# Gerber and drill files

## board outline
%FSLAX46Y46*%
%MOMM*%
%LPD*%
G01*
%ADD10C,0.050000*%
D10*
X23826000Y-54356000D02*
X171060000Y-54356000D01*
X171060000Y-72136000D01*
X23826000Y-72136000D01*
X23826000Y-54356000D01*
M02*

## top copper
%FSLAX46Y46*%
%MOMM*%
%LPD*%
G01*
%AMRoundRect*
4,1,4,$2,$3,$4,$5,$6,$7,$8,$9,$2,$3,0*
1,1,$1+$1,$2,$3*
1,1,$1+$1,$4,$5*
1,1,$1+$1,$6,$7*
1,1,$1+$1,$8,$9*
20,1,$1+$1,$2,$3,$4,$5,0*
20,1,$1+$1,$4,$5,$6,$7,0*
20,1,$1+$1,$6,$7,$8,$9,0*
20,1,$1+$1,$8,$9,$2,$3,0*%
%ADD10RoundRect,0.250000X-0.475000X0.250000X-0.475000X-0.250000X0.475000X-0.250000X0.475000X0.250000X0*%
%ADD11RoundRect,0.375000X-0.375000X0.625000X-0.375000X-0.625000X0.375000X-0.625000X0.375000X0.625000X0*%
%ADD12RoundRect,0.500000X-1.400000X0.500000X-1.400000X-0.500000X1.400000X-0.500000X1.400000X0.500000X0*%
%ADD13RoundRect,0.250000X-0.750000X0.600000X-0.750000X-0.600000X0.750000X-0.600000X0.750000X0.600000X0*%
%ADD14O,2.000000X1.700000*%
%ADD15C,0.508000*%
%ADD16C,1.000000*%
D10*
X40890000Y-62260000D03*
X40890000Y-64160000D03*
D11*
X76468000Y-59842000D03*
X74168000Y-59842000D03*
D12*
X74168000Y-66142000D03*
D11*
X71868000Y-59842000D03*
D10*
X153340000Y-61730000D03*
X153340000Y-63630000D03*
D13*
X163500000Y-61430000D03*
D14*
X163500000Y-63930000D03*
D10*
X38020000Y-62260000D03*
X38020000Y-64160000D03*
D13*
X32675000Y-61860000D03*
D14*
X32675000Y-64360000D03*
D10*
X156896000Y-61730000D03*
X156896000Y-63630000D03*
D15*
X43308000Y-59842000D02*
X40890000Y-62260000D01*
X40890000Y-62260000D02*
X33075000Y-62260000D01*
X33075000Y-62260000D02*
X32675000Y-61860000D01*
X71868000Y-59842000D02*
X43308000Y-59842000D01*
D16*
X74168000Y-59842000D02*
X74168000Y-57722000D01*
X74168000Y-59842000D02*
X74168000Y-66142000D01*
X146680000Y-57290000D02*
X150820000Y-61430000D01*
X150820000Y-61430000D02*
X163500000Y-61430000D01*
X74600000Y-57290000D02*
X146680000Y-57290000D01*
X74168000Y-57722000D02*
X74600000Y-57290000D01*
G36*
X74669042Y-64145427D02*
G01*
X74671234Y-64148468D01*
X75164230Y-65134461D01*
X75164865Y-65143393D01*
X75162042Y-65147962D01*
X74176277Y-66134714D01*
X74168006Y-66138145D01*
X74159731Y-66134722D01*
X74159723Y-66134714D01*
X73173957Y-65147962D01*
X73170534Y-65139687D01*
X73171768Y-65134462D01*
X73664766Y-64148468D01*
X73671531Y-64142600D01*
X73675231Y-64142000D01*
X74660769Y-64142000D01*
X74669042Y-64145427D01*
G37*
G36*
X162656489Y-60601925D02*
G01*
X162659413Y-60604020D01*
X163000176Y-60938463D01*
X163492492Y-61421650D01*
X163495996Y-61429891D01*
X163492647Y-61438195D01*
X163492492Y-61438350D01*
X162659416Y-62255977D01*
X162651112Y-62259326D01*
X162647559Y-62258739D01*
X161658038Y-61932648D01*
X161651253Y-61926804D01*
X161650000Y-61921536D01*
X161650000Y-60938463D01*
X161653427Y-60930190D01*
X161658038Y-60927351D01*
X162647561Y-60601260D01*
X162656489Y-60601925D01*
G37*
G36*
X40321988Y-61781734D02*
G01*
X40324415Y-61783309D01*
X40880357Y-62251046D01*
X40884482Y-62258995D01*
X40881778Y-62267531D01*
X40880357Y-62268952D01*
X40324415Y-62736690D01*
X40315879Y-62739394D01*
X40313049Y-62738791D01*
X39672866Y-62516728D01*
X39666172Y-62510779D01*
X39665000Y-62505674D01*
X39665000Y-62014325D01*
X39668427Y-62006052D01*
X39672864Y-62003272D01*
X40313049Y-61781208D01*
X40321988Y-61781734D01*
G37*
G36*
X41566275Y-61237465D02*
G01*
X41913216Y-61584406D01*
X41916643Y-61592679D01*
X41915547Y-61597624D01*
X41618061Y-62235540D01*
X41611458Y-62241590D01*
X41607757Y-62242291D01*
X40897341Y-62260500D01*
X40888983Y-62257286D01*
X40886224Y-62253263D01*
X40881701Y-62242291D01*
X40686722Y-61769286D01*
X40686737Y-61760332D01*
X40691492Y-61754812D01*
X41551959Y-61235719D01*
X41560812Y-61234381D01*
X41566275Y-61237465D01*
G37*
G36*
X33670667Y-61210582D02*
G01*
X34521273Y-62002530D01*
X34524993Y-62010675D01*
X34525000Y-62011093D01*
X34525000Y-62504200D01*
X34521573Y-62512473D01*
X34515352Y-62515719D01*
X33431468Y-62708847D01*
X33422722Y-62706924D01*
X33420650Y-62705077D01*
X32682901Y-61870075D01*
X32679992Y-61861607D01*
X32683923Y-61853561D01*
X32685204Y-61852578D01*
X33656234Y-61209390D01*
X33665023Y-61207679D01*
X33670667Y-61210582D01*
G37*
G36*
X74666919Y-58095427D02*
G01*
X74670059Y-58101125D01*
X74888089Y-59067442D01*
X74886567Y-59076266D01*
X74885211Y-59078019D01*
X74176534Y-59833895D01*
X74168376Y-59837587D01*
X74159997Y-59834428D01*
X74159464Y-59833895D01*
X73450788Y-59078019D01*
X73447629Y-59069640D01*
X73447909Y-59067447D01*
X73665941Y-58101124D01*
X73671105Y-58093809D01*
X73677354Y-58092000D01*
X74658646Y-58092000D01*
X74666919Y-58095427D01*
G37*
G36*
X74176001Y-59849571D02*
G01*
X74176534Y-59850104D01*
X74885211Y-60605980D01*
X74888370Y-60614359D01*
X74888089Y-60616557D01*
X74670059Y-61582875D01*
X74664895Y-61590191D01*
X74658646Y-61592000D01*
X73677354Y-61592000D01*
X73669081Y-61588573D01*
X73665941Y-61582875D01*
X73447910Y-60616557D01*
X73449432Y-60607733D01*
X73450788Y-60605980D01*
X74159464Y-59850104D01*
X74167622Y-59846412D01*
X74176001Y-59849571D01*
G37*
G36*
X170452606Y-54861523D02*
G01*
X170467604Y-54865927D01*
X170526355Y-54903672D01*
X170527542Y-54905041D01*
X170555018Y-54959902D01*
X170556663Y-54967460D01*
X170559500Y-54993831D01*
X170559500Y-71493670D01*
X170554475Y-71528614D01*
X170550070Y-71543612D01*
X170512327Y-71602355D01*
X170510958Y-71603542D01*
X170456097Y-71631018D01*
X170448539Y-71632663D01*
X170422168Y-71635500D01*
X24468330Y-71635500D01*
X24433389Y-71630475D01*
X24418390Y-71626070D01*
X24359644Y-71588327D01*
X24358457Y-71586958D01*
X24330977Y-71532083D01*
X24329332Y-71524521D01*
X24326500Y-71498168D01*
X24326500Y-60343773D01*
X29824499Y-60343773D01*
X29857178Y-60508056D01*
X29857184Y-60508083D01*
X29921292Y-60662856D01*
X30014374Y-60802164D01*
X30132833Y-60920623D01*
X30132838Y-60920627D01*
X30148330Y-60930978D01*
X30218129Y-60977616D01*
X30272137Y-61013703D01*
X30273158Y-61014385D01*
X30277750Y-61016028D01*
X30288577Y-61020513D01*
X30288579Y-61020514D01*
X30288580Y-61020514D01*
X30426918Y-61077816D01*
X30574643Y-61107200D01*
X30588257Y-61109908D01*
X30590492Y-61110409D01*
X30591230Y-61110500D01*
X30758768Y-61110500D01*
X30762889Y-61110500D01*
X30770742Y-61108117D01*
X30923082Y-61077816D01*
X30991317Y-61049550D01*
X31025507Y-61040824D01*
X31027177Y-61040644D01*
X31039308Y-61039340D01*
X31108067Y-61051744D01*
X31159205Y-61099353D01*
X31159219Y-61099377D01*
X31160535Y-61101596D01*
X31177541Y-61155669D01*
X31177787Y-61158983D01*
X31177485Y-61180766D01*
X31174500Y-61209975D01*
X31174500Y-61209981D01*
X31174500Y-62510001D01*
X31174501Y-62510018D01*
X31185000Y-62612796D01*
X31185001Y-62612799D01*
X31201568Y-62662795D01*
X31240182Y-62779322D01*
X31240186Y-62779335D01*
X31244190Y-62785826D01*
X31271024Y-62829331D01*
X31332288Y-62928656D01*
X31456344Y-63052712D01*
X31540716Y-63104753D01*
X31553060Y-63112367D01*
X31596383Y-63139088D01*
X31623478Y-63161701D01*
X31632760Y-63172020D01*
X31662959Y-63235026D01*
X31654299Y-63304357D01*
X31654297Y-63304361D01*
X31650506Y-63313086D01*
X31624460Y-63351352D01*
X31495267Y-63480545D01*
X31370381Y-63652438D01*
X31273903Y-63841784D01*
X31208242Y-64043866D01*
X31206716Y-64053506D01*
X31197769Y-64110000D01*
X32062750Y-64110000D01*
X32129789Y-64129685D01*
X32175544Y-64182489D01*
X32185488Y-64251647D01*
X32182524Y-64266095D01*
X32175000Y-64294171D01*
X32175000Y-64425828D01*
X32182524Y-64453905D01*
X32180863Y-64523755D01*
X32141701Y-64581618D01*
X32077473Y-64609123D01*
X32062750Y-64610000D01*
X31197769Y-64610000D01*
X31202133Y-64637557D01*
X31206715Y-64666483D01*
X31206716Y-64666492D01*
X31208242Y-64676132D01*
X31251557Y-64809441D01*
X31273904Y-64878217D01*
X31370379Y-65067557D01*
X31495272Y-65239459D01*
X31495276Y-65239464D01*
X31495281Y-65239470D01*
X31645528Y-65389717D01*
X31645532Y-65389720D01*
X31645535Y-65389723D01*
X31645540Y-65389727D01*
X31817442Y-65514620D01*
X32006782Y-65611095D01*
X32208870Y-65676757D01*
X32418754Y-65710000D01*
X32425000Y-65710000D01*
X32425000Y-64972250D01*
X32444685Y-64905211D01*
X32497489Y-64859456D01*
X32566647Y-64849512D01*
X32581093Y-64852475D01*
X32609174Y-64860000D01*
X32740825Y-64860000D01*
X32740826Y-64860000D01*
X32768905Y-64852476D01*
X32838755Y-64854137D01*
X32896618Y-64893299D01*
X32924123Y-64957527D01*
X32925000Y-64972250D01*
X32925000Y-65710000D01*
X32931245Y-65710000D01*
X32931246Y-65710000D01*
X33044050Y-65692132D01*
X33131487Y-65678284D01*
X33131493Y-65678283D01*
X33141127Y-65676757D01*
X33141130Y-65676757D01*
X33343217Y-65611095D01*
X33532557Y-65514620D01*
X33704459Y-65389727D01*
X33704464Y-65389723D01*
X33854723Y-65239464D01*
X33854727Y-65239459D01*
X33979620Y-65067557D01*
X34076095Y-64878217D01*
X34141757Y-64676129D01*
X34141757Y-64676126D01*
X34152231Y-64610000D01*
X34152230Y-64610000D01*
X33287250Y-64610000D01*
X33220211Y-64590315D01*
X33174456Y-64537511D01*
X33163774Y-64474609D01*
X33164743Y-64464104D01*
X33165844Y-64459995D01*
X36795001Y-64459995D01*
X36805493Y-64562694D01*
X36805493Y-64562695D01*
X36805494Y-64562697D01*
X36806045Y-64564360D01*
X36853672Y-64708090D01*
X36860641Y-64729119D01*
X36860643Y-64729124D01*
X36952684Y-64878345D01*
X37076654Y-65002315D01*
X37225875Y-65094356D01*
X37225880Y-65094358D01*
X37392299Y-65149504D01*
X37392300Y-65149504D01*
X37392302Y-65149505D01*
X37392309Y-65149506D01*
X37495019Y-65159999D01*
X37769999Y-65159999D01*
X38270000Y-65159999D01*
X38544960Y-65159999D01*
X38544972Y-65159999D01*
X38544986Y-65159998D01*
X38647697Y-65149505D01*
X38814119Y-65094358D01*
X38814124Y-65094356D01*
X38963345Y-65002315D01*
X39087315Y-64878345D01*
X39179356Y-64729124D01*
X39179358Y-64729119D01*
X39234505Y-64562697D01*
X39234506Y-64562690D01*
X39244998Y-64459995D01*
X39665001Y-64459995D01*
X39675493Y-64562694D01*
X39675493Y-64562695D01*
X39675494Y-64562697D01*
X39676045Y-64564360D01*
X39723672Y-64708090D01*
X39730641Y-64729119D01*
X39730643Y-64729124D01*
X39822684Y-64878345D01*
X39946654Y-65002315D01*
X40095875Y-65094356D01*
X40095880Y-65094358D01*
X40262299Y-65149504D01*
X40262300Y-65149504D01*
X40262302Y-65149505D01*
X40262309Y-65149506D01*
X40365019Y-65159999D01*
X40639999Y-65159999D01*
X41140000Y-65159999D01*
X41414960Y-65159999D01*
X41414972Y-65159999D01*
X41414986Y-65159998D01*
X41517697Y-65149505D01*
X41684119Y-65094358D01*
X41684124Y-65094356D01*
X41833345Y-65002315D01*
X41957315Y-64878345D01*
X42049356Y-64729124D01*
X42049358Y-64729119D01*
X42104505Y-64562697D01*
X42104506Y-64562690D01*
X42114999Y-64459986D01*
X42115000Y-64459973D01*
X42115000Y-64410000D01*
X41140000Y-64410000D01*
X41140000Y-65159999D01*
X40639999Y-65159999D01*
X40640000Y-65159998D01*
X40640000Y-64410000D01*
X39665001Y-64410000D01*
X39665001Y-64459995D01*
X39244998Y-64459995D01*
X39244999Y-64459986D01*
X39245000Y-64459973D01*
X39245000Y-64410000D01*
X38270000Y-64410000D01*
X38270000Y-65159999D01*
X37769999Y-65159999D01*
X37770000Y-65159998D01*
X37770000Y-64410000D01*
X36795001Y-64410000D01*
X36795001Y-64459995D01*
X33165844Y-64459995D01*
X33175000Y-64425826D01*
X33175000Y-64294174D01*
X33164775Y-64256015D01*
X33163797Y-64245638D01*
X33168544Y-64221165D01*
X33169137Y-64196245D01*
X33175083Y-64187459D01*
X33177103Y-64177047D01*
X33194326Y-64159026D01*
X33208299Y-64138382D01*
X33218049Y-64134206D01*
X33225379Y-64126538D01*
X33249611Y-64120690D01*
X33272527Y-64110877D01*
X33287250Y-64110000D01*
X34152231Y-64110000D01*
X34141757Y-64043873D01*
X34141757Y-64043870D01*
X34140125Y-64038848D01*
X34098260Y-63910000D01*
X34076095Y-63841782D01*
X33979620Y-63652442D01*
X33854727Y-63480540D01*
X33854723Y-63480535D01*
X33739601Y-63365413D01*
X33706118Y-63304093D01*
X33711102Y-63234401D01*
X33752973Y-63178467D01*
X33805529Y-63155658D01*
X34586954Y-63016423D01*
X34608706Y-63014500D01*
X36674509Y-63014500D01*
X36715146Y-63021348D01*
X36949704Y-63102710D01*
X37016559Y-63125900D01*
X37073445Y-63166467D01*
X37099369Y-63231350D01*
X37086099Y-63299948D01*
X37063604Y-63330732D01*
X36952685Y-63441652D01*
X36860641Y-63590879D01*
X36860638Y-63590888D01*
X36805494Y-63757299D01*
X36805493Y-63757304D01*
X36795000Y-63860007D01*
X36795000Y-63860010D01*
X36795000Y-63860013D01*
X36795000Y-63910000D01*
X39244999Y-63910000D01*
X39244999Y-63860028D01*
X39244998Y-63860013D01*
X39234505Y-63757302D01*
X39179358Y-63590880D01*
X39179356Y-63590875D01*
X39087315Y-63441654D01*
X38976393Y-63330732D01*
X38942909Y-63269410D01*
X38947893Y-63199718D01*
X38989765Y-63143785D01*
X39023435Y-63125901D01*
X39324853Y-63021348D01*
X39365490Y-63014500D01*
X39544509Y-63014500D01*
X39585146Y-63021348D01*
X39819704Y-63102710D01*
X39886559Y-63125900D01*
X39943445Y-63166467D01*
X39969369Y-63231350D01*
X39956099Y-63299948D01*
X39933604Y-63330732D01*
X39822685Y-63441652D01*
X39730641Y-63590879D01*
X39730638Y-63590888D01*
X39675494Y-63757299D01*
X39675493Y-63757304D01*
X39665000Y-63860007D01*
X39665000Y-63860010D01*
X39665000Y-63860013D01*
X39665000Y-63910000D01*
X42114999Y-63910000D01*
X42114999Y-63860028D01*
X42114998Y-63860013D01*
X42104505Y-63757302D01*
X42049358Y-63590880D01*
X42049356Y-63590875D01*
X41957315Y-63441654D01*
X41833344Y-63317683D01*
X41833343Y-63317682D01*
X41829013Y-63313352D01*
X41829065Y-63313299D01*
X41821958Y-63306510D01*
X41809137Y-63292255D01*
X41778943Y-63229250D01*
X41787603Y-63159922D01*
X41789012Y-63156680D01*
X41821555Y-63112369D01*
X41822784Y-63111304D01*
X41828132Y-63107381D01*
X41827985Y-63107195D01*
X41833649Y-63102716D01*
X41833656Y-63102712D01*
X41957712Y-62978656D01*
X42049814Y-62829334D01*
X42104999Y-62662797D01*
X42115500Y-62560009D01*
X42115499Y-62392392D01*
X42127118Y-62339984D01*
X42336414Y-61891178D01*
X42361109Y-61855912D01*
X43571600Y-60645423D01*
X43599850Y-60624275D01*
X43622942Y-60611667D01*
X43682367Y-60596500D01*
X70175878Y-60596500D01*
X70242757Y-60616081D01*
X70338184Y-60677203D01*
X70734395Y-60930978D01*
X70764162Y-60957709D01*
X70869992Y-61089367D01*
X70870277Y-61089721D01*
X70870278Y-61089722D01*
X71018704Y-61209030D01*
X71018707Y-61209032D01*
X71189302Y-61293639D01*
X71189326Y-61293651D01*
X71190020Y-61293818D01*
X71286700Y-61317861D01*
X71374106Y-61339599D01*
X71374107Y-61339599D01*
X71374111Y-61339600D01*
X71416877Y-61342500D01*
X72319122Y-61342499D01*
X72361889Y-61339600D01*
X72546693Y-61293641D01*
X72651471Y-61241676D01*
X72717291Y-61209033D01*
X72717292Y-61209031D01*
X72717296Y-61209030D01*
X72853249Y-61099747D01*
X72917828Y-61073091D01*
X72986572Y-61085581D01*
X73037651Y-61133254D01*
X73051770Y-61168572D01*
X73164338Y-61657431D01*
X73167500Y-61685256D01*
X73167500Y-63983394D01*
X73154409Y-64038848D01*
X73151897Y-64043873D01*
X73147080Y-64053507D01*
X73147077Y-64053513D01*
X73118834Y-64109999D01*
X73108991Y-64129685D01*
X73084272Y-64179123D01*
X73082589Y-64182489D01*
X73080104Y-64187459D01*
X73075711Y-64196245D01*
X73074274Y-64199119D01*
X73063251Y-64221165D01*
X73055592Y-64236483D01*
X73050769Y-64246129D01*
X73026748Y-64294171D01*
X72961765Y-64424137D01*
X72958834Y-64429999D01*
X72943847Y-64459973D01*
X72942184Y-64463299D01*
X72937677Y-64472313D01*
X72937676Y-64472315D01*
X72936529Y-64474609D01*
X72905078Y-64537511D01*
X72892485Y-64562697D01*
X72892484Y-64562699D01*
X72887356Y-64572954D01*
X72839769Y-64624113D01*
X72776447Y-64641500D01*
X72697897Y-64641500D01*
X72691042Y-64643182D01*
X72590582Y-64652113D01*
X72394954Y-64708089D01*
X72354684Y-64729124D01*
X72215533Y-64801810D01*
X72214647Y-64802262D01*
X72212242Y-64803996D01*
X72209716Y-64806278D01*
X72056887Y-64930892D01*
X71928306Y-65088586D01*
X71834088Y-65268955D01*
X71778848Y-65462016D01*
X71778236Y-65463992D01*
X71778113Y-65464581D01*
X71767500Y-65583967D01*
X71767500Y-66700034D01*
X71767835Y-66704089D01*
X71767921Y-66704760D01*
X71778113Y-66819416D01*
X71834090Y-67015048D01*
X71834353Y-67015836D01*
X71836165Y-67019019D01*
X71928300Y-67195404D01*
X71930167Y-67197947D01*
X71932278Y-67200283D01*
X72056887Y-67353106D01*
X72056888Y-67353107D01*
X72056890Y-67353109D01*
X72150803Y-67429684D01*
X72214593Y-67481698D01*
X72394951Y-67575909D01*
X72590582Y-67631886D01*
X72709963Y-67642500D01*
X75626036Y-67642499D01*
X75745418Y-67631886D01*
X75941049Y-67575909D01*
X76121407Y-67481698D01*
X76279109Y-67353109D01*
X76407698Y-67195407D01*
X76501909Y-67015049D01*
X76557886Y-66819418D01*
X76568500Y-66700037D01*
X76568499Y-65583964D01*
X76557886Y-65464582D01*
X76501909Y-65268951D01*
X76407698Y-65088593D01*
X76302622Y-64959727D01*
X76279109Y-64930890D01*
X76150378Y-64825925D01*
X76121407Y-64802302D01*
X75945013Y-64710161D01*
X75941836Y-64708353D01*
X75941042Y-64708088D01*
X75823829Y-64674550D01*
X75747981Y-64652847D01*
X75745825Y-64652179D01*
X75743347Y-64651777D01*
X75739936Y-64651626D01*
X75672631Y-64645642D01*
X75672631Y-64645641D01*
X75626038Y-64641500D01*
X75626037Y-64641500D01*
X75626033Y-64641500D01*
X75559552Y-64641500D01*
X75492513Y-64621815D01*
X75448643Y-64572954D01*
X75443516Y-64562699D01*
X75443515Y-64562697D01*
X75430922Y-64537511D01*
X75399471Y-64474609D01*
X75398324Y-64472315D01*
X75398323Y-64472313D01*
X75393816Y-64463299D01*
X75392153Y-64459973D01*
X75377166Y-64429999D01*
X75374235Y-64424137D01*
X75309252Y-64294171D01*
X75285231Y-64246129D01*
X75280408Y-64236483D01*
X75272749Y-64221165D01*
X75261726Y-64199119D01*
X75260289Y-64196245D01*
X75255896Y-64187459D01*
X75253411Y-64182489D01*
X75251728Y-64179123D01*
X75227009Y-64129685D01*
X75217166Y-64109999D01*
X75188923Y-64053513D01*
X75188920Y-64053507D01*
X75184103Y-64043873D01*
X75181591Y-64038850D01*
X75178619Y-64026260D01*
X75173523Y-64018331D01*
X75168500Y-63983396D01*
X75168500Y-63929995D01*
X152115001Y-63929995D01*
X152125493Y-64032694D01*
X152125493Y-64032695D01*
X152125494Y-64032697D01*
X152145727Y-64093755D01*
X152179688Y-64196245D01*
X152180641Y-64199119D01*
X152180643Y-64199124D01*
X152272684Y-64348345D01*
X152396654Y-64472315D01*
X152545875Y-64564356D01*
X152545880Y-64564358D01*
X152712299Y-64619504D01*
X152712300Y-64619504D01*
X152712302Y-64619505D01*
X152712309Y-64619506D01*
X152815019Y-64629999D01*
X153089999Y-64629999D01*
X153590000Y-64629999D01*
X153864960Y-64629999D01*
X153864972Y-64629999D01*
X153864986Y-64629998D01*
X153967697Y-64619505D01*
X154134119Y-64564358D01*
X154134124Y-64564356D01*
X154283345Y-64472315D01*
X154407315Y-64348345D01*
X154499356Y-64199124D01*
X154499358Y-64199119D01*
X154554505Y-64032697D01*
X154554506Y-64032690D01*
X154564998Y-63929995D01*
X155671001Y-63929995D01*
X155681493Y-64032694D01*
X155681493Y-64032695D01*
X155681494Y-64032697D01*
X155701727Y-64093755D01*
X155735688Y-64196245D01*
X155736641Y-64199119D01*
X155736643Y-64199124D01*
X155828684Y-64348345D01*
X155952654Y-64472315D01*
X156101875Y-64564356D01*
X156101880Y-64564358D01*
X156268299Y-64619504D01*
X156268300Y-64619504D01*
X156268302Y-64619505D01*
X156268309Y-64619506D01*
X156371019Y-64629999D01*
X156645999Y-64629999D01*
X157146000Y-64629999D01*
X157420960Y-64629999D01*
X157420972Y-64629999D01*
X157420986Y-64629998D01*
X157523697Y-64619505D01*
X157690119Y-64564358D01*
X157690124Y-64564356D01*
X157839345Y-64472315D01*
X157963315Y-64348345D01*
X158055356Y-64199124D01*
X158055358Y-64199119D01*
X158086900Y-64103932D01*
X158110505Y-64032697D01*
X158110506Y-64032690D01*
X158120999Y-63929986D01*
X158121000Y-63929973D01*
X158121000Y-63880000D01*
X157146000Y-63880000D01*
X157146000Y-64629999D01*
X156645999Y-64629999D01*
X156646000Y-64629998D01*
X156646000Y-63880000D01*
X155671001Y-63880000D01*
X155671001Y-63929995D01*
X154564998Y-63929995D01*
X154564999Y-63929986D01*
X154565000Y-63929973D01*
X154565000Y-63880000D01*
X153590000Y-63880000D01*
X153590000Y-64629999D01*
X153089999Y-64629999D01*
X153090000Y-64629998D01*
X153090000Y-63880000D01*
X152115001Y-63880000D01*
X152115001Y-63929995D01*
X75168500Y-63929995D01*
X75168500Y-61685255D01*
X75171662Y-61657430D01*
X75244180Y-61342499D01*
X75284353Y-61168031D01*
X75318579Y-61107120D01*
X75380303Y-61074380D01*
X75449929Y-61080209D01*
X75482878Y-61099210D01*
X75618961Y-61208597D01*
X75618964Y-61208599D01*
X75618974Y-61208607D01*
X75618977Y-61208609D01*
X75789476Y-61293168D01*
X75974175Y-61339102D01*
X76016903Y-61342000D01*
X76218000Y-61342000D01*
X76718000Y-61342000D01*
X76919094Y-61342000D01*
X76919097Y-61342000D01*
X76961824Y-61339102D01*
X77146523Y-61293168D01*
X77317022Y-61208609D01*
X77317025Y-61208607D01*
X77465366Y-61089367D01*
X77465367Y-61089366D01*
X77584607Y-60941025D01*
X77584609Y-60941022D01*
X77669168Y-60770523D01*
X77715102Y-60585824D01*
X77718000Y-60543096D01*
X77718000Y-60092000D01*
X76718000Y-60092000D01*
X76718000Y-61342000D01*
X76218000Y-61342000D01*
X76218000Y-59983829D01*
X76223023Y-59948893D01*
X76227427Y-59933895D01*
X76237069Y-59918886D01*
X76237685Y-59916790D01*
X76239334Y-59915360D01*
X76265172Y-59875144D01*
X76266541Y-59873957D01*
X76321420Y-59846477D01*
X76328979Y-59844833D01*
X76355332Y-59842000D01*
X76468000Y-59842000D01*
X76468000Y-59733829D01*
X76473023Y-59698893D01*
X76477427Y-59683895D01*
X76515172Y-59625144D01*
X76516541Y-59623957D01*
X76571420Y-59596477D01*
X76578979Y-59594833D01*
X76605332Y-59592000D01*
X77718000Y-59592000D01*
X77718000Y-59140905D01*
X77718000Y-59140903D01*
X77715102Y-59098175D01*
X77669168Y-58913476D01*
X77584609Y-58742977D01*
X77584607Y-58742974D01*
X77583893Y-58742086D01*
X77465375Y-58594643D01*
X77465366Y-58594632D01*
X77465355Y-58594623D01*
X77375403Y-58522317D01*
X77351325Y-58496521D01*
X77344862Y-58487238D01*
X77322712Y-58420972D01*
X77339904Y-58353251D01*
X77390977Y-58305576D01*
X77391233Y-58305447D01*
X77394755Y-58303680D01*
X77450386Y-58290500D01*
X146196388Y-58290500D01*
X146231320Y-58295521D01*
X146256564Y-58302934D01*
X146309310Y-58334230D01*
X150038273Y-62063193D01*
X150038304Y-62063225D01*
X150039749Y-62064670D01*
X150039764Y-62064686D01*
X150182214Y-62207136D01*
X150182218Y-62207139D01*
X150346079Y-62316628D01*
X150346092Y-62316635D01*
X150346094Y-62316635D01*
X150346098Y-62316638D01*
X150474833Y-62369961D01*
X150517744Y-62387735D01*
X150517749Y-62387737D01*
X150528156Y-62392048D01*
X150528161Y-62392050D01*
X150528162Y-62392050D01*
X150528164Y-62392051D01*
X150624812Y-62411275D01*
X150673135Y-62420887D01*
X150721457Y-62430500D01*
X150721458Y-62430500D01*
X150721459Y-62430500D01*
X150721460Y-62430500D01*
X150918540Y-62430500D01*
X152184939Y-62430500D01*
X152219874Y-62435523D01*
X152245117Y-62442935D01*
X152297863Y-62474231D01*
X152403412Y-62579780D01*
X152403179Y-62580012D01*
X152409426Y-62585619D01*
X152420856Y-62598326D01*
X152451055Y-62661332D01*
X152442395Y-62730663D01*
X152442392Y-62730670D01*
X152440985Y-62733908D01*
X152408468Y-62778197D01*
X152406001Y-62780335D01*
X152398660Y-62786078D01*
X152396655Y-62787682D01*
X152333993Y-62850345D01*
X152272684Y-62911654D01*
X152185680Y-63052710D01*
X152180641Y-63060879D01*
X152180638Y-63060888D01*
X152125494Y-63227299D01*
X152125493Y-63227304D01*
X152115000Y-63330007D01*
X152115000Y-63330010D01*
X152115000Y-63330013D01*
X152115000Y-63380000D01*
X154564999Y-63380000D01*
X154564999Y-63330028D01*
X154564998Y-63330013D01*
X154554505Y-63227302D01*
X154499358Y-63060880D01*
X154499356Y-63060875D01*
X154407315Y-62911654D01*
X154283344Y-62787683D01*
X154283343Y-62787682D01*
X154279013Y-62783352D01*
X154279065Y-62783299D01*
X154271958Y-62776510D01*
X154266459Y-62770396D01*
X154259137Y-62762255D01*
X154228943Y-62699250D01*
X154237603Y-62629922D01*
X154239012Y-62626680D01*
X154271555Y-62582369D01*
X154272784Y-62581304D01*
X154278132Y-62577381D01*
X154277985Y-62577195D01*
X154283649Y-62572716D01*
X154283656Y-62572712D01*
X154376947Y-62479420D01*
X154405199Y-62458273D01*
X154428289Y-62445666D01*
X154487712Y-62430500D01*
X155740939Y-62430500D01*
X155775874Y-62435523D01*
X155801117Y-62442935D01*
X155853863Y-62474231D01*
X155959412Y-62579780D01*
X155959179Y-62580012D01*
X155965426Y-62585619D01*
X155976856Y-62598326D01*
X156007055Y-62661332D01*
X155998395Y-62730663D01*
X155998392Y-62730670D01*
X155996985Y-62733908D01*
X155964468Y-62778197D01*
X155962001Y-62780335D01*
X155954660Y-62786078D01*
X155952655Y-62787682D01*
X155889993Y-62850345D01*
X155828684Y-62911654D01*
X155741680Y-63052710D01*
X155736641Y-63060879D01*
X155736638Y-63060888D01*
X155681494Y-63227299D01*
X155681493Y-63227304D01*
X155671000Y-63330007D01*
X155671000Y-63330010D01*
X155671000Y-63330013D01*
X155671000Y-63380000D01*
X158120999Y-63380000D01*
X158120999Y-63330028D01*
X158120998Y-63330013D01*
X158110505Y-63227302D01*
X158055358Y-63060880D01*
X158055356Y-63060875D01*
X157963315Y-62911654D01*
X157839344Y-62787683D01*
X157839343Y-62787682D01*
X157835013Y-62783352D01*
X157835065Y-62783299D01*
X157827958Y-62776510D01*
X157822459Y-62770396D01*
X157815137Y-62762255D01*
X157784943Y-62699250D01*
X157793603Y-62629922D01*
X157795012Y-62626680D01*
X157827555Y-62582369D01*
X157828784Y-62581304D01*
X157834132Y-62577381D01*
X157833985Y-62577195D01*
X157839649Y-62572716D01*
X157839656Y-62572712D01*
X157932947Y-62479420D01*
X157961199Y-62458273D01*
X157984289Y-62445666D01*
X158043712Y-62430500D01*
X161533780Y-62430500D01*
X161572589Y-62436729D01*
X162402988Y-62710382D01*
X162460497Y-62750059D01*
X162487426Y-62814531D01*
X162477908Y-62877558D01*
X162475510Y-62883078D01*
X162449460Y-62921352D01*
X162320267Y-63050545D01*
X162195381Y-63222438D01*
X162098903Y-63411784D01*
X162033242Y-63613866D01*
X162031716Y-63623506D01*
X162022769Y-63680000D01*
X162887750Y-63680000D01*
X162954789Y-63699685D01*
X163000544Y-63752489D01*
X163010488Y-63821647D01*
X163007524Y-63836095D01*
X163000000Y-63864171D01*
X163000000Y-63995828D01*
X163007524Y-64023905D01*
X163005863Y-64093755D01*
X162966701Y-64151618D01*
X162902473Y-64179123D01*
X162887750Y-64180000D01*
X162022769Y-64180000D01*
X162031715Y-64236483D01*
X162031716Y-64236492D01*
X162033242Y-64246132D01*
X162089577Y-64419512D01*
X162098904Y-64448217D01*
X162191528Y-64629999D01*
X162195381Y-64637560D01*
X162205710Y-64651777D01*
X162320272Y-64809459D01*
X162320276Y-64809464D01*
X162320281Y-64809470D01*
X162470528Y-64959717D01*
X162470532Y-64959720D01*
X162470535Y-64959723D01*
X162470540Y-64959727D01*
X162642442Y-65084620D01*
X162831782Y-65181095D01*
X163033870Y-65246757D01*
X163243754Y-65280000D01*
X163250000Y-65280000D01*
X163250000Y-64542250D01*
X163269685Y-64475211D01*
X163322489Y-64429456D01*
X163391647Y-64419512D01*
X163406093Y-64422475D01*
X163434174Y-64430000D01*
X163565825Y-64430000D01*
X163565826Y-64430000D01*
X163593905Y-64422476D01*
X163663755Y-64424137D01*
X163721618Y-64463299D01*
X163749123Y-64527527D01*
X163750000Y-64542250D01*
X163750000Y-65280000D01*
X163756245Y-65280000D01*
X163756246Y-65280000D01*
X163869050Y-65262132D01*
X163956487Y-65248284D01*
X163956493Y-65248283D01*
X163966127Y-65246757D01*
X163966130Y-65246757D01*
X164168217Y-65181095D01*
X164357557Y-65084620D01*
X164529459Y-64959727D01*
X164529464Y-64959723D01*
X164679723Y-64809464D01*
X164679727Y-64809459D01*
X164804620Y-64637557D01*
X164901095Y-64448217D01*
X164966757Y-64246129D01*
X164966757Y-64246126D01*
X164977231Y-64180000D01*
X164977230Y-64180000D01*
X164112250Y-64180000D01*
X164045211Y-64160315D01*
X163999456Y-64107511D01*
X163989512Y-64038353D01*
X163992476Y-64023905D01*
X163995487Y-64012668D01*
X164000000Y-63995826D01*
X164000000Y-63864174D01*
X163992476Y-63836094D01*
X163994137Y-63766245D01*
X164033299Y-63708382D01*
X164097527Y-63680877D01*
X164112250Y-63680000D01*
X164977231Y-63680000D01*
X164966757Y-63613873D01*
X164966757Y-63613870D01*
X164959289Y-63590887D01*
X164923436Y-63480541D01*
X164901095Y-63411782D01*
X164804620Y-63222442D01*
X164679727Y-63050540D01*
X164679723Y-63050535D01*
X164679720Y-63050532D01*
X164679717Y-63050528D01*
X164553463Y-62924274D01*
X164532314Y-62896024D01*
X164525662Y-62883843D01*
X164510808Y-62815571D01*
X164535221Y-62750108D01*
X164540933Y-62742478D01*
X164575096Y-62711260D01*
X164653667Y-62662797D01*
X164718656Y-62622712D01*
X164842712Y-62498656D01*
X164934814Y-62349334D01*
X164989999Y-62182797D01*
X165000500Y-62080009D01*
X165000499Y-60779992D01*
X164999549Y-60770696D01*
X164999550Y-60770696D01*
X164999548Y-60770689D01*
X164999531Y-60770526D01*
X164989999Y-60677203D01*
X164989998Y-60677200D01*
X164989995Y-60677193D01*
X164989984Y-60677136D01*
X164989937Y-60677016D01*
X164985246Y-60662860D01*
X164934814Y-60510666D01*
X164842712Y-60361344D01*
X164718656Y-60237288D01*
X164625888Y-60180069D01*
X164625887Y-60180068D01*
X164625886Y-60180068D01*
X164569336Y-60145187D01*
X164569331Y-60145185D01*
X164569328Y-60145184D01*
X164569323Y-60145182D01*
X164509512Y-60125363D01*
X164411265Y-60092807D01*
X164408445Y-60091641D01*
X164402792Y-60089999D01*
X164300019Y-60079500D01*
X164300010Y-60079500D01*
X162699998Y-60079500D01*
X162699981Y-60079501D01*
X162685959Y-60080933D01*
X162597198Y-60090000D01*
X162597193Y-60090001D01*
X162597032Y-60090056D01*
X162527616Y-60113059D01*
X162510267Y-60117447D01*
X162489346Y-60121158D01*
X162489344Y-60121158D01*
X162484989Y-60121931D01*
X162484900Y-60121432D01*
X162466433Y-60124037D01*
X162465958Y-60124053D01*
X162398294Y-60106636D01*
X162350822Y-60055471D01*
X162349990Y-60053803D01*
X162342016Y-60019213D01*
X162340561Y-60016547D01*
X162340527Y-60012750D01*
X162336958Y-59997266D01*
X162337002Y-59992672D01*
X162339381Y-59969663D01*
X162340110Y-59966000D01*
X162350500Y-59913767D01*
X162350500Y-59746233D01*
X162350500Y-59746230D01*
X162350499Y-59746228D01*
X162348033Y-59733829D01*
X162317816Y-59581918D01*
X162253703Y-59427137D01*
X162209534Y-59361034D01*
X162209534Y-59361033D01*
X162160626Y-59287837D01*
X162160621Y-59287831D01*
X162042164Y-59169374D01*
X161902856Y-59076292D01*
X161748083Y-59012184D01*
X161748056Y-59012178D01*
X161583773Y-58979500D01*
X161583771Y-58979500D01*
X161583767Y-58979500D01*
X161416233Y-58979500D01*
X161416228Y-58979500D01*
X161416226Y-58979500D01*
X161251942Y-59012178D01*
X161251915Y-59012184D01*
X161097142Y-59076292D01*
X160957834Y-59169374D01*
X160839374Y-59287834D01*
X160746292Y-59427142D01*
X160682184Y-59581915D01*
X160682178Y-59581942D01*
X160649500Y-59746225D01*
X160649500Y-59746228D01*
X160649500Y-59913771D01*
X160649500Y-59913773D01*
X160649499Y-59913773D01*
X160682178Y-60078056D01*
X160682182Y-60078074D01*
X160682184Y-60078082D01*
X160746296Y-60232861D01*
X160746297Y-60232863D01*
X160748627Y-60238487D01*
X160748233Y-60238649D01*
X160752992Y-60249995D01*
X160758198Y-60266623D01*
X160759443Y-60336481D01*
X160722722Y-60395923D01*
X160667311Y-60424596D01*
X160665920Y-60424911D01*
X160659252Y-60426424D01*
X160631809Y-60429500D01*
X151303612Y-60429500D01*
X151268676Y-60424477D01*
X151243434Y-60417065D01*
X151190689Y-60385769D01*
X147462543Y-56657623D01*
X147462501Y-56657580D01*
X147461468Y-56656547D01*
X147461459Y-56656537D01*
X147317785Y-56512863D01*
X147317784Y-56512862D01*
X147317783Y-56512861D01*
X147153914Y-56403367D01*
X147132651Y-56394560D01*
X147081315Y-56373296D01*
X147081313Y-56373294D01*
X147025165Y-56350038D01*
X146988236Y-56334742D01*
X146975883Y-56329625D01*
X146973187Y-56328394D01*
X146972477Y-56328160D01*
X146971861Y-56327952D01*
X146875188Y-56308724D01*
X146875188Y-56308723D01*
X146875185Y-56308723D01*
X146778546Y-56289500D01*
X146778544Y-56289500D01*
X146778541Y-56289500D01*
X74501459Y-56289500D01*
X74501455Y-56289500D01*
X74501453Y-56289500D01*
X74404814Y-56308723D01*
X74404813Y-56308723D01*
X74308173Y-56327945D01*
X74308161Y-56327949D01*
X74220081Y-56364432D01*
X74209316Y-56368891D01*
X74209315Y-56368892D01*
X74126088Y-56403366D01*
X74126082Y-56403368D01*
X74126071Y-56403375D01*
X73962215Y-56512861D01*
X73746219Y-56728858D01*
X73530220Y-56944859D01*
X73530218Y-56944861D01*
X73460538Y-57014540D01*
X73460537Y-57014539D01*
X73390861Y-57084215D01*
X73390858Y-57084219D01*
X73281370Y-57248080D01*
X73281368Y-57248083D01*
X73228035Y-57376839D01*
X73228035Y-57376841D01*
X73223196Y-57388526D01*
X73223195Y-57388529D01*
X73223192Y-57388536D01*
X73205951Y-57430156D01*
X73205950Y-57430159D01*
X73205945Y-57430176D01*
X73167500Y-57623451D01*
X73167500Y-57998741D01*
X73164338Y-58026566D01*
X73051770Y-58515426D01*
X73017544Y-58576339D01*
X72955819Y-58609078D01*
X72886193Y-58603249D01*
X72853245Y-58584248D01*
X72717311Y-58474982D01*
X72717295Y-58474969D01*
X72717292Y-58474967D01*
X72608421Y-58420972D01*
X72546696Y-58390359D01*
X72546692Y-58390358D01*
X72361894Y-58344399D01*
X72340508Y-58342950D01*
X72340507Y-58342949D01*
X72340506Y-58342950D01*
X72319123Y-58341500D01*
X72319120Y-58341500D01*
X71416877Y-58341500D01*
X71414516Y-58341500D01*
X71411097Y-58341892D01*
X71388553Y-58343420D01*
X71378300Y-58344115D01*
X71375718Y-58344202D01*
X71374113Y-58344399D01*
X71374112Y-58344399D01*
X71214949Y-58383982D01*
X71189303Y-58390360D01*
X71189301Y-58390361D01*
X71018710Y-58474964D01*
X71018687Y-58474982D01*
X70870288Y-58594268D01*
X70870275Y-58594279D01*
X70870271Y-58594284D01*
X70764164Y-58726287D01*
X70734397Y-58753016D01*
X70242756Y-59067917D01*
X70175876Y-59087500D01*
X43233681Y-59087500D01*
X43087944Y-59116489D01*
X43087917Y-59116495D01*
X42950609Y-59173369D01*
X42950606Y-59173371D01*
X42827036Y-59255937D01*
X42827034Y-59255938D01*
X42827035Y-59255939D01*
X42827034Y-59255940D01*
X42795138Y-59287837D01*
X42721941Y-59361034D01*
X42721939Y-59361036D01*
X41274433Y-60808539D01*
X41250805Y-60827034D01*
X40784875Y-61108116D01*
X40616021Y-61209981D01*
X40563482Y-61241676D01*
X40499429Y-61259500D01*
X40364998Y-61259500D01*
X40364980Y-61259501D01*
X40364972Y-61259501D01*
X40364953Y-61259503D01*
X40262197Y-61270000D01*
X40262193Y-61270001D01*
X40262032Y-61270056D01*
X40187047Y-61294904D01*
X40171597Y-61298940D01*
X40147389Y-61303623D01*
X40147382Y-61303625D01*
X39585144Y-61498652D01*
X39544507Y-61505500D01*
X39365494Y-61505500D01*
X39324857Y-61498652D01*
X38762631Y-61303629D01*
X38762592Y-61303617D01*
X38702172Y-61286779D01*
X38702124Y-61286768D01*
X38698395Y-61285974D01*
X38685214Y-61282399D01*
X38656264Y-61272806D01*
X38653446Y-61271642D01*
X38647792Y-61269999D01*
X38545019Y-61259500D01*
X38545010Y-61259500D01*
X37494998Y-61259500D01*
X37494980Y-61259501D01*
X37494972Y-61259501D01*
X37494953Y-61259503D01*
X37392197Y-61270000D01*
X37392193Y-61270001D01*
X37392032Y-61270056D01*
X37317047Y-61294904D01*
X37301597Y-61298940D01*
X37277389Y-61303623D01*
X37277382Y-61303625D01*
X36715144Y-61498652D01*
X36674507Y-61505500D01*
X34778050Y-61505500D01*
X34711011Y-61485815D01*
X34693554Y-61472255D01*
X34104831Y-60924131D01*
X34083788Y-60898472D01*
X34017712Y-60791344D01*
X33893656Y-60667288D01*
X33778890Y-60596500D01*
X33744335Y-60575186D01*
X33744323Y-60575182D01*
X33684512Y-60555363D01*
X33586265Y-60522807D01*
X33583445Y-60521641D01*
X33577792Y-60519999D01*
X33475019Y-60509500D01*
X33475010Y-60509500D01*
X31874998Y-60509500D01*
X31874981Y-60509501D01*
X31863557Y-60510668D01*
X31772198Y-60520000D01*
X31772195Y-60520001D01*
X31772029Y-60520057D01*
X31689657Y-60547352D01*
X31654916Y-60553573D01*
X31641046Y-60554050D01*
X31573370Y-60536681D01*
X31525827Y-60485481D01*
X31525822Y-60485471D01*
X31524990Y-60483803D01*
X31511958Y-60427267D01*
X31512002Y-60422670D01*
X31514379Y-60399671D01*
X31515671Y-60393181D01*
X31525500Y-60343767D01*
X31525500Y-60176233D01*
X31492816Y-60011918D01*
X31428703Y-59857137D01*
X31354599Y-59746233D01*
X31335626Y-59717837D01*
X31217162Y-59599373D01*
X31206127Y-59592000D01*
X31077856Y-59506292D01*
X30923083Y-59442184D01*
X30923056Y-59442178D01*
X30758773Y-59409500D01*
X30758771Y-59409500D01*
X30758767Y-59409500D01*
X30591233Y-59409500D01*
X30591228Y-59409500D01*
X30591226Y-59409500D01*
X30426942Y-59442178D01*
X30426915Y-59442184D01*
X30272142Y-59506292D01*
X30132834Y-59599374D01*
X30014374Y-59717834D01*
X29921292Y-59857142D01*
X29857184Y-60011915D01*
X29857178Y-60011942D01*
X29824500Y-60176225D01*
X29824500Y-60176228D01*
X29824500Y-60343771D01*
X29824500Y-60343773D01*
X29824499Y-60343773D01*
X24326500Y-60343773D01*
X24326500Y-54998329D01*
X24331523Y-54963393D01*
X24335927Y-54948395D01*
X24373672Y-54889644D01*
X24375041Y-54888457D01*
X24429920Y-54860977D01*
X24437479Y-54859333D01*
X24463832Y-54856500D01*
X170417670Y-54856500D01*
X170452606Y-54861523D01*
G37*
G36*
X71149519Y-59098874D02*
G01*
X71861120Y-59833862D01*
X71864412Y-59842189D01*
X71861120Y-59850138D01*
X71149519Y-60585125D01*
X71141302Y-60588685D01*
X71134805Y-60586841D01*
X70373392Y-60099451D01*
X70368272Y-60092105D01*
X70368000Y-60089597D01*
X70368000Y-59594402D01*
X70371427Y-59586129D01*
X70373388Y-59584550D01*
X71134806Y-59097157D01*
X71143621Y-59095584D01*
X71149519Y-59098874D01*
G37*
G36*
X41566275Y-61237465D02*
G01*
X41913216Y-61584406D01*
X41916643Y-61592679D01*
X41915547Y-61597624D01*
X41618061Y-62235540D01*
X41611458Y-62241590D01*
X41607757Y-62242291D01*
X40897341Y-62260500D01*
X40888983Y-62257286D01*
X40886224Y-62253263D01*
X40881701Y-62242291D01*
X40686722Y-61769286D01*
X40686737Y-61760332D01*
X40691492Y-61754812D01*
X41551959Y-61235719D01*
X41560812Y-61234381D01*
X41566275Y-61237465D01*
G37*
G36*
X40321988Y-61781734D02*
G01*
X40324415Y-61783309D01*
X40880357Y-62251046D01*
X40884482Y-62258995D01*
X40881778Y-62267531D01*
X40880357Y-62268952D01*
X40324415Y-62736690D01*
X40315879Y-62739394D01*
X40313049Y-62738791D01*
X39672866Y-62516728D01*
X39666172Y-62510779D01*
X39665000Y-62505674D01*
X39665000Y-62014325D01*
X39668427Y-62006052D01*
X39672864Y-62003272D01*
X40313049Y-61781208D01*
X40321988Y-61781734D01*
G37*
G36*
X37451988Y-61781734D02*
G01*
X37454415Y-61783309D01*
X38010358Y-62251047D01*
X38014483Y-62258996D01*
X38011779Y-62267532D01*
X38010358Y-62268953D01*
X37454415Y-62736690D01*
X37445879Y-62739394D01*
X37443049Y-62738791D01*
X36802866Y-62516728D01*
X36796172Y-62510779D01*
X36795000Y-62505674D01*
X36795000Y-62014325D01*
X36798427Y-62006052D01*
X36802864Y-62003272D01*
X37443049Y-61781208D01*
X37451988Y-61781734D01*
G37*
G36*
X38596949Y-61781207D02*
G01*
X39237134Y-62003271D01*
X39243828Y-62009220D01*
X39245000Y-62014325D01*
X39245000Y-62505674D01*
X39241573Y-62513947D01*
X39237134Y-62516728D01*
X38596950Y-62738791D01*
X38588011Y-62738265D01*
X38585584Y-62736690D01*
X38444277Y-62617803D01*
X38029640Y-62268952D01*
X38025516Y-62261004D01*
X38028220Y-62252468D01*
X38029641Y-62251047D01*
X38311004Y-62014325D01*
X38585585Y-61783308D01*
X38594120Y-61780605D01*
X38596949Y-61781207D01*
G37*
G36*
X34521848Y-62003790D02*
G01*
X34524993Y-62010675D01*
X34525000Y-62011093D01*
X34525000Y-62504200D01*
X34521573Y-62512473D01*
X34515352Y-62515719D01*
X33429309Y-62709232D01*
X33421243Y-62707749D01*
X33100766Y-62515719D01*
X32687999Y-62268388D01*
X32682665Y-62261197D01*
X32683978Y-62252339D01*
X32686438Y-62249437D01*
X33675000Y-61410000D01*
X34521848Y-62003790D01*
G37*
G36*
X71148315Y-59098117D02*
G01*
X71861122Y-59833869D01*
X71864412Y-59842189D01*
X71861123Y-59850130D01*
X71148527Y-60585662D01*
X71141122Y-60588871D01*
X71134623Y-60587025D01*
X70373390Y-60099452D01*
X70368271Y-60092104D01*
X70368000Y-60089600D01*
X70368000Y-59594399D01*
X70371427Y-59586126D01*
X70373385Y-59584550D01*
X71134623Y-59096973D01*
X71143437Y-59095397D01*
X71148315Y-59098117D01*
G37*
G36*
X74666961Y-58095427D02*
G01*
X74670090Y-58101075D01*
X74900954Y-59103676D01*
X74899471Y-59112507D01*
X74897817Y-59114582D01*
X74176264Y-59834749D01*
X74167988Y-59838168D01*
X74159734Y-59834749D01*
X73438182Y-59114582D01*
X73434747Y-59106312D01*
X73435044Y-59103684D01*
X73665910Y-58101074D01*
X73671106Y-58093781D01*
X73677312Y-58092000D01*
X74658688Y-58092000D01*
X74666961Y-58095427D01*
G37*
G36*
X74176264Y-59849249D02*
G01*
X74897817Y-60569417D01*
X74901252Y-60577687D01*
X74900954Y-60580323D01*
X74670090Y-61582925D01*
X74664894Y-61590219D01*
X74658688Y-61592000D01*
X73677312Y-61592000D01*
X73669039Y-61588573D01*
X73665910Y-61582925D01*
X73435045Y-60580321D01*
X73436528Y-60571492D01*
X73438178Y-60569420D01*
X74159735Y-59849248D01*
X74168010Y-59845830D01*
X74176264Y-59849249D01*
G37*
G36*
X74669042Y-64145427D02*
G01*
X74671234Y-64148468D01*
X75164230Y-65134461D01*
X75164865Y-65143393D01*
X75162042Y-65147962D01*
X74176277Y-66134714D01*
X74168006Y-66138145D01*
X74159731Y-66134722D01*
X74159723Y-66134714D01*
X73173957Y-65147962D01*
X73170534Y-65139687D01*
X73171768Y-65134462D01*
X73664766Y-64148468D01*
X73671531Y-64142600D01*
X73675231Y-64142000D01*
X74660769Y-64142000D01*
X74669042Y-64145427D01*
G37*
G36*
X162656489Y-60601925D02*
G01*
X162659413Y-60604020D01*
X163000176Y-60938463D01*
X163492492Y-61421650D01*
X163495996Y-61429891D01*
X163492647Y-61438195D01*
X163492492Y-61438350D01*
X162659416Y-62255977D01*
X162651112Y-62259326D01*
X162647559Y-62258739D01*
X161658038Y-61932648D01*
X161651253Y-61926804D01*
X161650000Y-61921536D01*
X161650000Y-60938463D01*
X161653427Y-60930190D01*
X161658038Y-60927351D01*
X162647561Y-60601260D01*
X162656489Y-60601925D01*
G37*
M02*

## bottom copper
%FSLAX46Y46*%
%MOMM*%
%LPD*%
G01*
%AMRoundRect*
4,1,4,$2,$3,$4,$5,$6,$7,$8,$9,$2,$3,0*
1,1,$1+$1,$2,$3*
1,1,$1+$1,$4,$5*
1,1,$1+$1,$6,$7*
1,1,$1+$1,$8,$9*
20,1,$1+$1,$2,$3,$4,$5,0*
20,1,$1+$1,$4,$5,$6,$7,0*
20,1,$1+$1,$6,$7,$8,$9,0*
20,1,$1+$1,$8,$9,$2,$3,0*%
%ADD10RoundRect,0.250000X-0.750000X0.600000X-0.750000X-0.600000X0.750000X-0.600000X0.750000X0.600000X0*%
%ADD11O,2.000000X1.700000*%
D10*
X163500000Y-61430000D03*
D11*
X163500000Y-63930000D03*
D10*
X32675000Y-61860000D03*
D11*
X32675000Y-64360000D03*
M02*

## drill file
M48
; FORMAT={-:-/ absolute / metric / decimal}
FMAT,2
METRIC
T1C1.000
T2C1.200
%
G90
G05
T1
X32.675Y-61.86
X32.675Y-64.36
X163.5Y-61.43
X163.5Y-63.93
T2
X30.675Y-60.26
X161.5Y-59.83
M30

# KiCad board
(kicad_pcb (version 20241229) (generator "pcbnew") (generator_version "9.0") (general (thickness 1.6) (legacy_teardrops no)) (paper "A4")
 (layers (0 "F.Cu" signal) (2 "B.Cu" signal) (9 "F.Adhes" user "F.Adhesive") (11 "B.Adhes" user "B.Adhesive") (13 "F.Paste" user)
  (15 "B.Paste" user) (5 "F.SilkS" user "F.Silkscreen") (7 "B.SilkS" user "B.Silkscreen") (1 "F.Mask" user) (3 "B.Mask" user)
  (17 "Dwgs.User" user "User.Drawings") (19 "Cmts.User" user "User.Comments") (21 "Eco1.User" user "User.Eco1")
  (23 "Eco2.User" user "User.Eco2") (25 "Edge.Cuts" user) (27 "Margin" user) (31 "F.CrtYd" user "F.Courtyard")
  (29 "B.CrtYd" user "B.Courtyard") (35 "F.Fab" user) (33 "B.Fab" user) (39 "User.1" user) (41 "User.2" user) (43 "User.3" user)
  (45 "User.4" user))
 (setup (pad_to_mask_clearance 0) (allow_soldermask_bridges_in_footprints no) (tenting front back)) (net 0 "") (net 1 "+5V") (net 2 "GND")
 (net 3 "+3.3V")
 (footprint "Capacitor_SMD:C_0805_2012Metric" (layer "F.Cu") (at 40.89 63.21 -90)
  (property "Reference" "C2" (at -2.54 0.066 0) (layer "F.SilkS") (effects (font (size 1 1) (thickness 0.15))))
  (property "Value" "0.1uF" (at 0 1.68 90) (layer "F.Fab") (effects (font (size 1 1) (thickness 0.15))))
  (pad "1" smd roundrect (at -0.95 0 270) (size 1 1.45) (layers "F.Cu" "F.Mask" "F.Paste") (roundrect_rratio 0.25) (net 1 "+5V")
   (teardrops (best_length_ratio 0.5) (max_length 1) (best_width_ratio 1) (max_width 2) (curved_edges no) (filter_ratio 0.9) (enabled yes)
    (allow_two_segments yes) (prefer_zone_connections yes)))
  (pad "2" smd roundrect (at 0.95 0 270) (size 1 1.45) (layers "F.Cu" "F.Mask" "F.Paste") (roundrect_rratio 0.25) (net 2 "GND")
   (teardrops (best_length_ratio 0.5) (max_length 1) (best_width_ratio 1) (max_width 2) (curved_edges no) (filter_ratio 0.9) (enabled yes)
    (allow_two_segments yes) (prefer_zone_connections yes))))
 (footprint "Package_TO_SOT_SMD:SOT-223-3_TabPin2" (layer "F.Cu") (at 74.168 62.992 -90)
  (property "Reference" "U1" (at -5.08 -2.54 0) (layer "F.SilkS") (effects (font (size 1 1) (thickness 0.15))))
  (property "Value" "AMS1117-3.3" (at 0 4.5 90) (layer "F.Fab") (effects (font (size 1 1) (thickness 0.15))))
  (pad "1" smd roundrect (at -3.15 -2.3 270) (size 2 1.5) (layers "F.Cu" "F.Mask" "F.Paste") (roundrect_rratio 0.25) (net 2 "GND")
   (teardrops (best_length_ratio 0.5) (max_length 1) (best_width_ratio 1) (max_width 2) (curved_edges no) (filter_ratio 0.9) (enabled yes)
    (allow_two_segments yes) (prefer_zone_connections yes)))
  (pad "2" smd roundrect (at -3.15 0 270) (size 2 1.5) (layers "F.Cu" "F.Mask" "F.Paste") (roundrect_rratio 0.25) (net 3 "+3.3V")
   (teardrops (best_length_ratio 0.5) (max_length 1) (best_width_ratio 1) (max_width 2) (curved_edges no) (filter_ratio 0.9) (enabled yes)
    (allow_two_segments yes) (prefer_zone_connections yes)))
  (pad "2" smd roundrect (at 3.15 0 270) (size 2 3.8) (layers "F.Cu" "F.Mask" "F.Paste") (roundrect_rratio 0.25) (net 3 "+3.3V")
   (teardrops (best_length_ratio 0.5) (max_length 1) (best_width_ratio 1) (max_width 2) (curved_edges no) (filter_ratio 0.9) (enabled yes)
    (allow_two_segments yes) (prefer_zone_connections yes)))
  (pad "3" smd roundrect (at -3.15 2.3 270) (size 2 1.5) (layers "F.Cu" "F.Mask" "F.Paste") (roundrect_rratio 0.25) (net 1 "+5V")
   (teardrops (best_length_ratio 0.5) (max_length 1) (best_width_ratio 1) (max_width 2) (curved_edges no) (filter_ratio 0.9) (enabled yes)
    (allow_two_segments yes) (prefer_zone_connections yes))))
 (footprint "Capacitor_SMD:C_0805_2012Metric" (layer "F.Cu") (at 153.34 62.68 -90)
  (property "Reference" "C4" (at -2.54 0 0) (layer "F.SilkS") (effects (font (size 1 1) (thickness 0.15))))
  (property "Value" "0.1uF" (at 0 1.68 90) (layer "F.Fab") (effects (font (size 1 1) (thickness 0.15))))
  (pad "1" smd roundrect (at -0.95 0 270) (size 1 1.45) (layers "F.Cu" "F.Mask" "F.Paste") (roundrect_rratio 0.25) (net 3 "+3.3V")
   (teardrops (best_length_ratio 0.5) (max_length 1) (best_width_ratio 1) (max_width 2) (curved_edges no) (filter_ratio 0.9) (enabled yes)
    (allow_two_segments yes) (prefer_zone_connections yes)))
  (pad "2" smd roundrect (at 0.95 0 270) (size 1 1.45) (layers "F.Cu" "F.Mask" "F.Paste") (roundrect_rratio 0.25) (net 2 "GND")
   (teardrops (best_length_ratio 0.5) (max_length 1) (best_width_ratio 1) (max_width 2) (curved_edges no) (filter_ratio 0.9) (enabled yes)
    (allow_two_segments yes) (prefer_zone_connections yes))))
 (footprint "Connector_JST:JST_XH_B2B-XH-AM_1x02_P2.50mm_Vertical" (layer "F.Cu") (at 163.5 61.43 -90)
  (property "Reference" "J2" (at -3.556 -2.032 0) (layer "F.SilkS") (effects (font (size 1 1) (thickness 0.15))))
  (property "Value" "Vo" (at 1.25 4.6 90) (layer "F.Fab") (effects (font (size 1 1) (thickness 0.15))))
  (pad "" np_thru_hole circle (at -1.6 2 270) (size 1.2 1.2) (drill 1.2) (layers "*.Cu" "*.Mask"))
  (pad "1" thru_hole roundrect (at 0 0 270) (size 1.7 2) (drill 1) (layers "*.Cu" "*.Mask") (remove_unused_layers no)
   (roundrect_rratio 0.147059) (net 3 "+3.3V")
   (teardrops (best_length_ratio 0.5) (max_length 1) (best_width_ratio 1) (max_width 2) (curved_edges no) (filter_ratio 0.9) (enabled yes)
    (allow_two_segments yes) (prefer_zone_connections yes)))
  (pad "2" thru_hole oval (at 2.5 0 270) (size 1.7 2) (drill 1) (layers "*.Cu" "*.Mask") (remove_unused_layers no) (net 2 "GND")
   (teardrops (best_length_ratio 0.5) (max_length 1) (best_width_ratio 1) (max_width 2) (curved_edges no) (filter_ratio 0.9) (enabled yes)
    (allow_two_segments yes) (prefer_zone_connections yes))))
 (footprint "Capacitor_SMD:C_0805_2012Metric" (layer "F.Cu") (at 38.02 63.21 -90)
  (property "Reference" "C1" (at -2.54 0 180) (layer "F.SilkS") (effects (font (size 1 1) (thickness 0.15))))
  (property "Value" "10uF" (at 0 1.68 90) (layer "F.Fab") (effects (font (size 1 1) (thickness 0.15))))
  (pad "1" smd roundrect (at -0.95 0 270) (size 1 1.45) (layers "F.Cu" "F.Mask" "F.Paste") (roundrect_rratio 0.25) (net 1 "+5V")
   (teardrops (best_length_ratio 0.5) (max_length 1) (best_width_ratio 1) (max_width 2) (curved_edges no) (filter_ratio 0.9) (enabled yes)
    (allow_two_segments yes) (prefer_zone_connections yes)))
  (pad "2" smd roundrect (at 0.95 0 270) (size 1 1.45) (layers "F.Cu" "F.Mask" "F.Paste") (roundrect_rratio 0.25) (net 2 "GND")
   (teardrops (best_length_ratio 0.5) (max_length 1) (best_width_ratio 1) (max_width 2) (curved_edges no) (filter_ratio 0.9) (enabled yes)
    (allow_two_segments yes) (prefer_zone_connections yes))))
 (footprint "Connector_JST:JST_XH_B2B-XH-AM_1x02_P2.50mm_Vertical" (layer "F.Cu") (at 32.675 61.86 -90)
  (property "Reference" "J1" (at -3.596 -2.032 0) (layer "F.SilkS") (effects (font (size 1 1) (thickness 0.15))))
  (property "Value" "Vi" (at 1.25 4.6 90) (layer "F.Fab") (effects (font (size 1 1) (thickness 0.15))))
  (pad "" np_thru_hole circle (at -1.6 2 270) (size 1.2 1.2) (drill 1.2) (layers "*.Cu" "*.Mask"))
  (pad "1" thru_hole roundrect (at 0 0 270) (size 1.7 2) (drill 1) (layers "*.Cu" "*.Mask") (remove_unused_layers no)
   (roundrect_rratio 0.147059) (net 1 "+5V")
   (teardrops (best_length_ratio 0.5) (max_length 1) (best_width_ratio 1) (max_width 2) (curved_edges no) (filter_ratio 0.9) (enabled yes)
    (allow_two_segments yes) (prefer_zone_connections yes)))
  (pad "2" thru_hole oval (at 2.5 0 270) (size 1.7 2) (drill 1) (layers "*.Cu" "*.Mask") (remove_unused_layers no) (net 2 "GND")
   (teardrops (best_length_ratio 0.5) (max_length 1) (best_width_ratio 1) (max_width 2) (curved_edges no) (filter_ratio 0.9) (enabled yes)
    (allow_two_segments yes) (prefer_zone_connections yes))))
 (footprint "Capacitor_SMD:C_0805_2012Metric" (layer "F.Cu") (at 156.896 62.68 -90)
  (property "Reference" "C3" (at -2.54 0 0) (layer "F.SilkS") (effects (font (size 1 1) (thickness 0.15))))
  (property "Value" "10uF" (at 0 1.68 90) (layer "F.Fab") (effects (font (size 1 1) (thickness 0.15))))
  (pad "1" smd roundrect (at -0.95 0 270) (size 1 1.45) (layers "F.Cu" "F.Mask" "F.Paste") (roundrect_rratio 0.25) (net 3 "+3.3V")
   (teardrops (best_length_ratio 0.5) (max_length 1) (best_width_ratio 1) (max_width 2) (curved_edges no) (filter_ratio 0.9) (enabled yes)
    (allow_two_segments yes) (prefer_zone_connections yes)))
  (pad "2" smd roundrect (at 0.95 0 270) (size 1 1.45) (layers "F.Cu" "F.Mask" "F.Paste") (roundrect_rratio 0.25) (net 2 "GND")
   (teardrops (best_length_ratio 0.5) (max_length 1) (best_width_ratio 1) (max_width 2) (curved_edges no) (filter_ratio 0.9) (enabled yes)
    (allow_two_segments yes) (prefer_zone_connections yes))))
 (gr_rect (start 23.826 54.356) (end 171.06 72.136) (stroke (width 0.05) (type default)) (fill no) (layer "Edge.Cuts"))
 (segment (start 43.308 59.842) (end 40.89 62.26) (width 0.508) (layer "F.Cu") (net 1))
 (segment (start 40.89 62.26) (end 33.075 62.26) (width 0.508) (layer "F.Cu") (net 1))
 (segment (start 33.075 62.26) (end 32.675 61.86) (width 0.508) (layer "F.Cu") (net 1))
 (segment (start 71.868 59.842) (end 43.308 59.842) (width 0.508) (layer "F.Cu") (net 1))
 (segment (start 74.168 59.842) (end 74.168 57.722) (width 1) (layer "F.Cu") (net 3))
 (segment (start 74.168 59.842) (end 74.168 66.142) (width 1) (layer "F.Cu") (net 3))
 (segment (start 146.68 57.29) (end 150.82 61.43) (width 1) (layer "F.Cu") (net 3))
 (segment (start 150.82 61.43) (end 163.5 61.43) (width 1) (layer "F.Cu") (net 3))
 (segment (start 74.6 57.29) (end 146.68 57.29) (width 1) (layer "F.Cu") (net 3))
 (segment (start 74.168 57.722) (end 74.6 57.29) (width 1) (layer "F.Cu") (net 3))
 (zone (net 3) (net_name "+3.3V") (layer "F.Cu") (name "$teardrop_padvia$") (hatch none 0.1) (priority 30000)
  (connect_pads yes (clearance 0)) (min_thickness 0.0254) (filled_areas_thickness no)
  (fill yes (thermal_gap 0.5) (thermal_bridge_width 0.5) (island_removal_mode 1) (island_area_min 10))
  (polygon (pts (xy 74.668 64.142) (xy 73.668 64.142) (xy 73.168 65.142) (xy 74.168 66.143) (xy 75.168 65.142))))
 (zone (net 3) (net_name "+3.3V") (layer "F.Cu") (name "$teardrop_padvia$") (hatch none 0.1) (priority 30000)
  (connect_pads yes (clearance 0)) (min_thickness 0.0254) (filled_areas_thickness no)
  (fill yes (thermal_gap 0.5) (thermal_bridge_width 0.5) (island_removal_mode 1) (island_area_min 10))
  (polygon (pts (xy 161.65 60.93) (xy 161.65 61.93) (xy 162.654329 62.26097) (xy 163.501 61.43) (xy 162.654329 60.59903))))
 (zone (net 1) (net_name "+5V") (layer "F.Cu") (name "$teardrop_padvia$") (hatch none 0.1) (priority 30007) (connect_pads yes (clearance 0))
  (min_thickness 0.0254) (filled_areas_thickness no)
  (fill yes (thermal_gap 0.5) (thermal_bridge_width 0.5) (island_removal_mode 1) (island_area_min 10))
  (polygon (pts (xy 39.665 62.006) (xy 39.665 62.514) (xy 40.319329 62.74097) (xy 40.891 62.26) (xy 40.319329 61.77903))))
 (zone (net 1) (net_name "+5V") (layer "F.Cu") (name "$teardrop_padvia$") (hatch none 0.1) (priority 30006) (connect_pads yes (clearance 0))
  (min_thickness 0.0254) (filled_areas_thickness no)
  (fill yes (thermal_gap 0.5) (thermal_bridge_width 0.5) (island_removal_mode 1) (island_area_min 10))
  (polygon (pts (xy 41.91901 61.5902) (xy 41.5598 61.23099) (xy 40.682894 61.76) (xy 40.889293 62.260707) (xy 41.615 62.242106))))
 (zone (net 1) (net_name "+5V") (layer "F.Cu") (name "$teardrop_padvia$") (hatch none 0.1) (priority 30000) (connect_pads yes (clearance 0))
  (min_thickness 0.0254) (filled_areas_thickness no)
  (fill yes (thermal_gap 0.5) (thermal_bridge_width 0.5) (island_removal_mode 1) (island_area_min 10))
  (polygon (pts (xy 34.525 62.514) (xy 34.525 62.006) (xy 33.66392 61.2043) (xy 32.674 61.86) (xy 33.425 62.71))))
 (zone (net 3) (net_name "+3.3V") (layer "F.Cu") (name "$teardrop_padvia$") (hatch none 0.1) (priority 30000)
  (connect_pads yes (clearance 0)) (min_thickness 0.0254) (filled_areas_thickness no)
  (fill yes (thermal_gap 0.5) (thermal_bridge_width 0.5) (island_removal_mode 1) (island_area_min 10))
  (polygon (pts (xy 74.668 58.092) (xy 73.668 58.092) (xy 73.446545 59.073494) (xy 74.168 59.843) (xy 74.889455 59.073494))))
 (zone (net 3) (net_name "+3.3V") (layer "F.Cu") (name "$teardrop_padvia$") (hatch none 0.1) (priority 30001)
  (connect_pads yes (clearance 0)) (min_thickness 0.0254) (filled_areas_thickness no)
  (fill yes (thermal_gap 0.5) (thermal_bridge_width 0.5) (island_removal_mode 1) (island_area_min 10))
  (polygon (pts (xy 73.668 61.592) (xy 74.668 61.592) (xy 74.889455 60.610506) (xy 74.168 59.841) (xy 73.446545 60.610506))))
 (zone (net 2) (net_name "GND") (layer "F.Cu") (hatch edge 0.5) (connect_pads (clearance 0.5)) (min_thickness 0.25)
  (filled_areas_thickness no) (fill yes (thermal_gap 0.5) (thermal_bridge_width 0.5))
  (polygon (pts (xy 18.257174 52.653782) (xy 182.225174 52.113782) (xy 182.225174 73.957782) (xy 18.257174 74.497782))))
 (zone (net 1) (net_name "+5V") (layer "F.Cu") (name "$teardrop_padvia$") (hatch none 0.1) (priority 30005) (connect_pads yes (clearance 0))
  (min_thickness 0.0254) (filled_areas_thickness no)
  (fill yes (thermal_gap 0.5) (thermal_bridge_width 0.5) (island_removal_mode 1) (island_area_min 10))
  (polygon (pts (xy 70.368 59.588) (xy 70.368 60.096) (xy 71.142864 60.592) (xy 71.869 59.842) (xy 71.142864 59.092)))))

